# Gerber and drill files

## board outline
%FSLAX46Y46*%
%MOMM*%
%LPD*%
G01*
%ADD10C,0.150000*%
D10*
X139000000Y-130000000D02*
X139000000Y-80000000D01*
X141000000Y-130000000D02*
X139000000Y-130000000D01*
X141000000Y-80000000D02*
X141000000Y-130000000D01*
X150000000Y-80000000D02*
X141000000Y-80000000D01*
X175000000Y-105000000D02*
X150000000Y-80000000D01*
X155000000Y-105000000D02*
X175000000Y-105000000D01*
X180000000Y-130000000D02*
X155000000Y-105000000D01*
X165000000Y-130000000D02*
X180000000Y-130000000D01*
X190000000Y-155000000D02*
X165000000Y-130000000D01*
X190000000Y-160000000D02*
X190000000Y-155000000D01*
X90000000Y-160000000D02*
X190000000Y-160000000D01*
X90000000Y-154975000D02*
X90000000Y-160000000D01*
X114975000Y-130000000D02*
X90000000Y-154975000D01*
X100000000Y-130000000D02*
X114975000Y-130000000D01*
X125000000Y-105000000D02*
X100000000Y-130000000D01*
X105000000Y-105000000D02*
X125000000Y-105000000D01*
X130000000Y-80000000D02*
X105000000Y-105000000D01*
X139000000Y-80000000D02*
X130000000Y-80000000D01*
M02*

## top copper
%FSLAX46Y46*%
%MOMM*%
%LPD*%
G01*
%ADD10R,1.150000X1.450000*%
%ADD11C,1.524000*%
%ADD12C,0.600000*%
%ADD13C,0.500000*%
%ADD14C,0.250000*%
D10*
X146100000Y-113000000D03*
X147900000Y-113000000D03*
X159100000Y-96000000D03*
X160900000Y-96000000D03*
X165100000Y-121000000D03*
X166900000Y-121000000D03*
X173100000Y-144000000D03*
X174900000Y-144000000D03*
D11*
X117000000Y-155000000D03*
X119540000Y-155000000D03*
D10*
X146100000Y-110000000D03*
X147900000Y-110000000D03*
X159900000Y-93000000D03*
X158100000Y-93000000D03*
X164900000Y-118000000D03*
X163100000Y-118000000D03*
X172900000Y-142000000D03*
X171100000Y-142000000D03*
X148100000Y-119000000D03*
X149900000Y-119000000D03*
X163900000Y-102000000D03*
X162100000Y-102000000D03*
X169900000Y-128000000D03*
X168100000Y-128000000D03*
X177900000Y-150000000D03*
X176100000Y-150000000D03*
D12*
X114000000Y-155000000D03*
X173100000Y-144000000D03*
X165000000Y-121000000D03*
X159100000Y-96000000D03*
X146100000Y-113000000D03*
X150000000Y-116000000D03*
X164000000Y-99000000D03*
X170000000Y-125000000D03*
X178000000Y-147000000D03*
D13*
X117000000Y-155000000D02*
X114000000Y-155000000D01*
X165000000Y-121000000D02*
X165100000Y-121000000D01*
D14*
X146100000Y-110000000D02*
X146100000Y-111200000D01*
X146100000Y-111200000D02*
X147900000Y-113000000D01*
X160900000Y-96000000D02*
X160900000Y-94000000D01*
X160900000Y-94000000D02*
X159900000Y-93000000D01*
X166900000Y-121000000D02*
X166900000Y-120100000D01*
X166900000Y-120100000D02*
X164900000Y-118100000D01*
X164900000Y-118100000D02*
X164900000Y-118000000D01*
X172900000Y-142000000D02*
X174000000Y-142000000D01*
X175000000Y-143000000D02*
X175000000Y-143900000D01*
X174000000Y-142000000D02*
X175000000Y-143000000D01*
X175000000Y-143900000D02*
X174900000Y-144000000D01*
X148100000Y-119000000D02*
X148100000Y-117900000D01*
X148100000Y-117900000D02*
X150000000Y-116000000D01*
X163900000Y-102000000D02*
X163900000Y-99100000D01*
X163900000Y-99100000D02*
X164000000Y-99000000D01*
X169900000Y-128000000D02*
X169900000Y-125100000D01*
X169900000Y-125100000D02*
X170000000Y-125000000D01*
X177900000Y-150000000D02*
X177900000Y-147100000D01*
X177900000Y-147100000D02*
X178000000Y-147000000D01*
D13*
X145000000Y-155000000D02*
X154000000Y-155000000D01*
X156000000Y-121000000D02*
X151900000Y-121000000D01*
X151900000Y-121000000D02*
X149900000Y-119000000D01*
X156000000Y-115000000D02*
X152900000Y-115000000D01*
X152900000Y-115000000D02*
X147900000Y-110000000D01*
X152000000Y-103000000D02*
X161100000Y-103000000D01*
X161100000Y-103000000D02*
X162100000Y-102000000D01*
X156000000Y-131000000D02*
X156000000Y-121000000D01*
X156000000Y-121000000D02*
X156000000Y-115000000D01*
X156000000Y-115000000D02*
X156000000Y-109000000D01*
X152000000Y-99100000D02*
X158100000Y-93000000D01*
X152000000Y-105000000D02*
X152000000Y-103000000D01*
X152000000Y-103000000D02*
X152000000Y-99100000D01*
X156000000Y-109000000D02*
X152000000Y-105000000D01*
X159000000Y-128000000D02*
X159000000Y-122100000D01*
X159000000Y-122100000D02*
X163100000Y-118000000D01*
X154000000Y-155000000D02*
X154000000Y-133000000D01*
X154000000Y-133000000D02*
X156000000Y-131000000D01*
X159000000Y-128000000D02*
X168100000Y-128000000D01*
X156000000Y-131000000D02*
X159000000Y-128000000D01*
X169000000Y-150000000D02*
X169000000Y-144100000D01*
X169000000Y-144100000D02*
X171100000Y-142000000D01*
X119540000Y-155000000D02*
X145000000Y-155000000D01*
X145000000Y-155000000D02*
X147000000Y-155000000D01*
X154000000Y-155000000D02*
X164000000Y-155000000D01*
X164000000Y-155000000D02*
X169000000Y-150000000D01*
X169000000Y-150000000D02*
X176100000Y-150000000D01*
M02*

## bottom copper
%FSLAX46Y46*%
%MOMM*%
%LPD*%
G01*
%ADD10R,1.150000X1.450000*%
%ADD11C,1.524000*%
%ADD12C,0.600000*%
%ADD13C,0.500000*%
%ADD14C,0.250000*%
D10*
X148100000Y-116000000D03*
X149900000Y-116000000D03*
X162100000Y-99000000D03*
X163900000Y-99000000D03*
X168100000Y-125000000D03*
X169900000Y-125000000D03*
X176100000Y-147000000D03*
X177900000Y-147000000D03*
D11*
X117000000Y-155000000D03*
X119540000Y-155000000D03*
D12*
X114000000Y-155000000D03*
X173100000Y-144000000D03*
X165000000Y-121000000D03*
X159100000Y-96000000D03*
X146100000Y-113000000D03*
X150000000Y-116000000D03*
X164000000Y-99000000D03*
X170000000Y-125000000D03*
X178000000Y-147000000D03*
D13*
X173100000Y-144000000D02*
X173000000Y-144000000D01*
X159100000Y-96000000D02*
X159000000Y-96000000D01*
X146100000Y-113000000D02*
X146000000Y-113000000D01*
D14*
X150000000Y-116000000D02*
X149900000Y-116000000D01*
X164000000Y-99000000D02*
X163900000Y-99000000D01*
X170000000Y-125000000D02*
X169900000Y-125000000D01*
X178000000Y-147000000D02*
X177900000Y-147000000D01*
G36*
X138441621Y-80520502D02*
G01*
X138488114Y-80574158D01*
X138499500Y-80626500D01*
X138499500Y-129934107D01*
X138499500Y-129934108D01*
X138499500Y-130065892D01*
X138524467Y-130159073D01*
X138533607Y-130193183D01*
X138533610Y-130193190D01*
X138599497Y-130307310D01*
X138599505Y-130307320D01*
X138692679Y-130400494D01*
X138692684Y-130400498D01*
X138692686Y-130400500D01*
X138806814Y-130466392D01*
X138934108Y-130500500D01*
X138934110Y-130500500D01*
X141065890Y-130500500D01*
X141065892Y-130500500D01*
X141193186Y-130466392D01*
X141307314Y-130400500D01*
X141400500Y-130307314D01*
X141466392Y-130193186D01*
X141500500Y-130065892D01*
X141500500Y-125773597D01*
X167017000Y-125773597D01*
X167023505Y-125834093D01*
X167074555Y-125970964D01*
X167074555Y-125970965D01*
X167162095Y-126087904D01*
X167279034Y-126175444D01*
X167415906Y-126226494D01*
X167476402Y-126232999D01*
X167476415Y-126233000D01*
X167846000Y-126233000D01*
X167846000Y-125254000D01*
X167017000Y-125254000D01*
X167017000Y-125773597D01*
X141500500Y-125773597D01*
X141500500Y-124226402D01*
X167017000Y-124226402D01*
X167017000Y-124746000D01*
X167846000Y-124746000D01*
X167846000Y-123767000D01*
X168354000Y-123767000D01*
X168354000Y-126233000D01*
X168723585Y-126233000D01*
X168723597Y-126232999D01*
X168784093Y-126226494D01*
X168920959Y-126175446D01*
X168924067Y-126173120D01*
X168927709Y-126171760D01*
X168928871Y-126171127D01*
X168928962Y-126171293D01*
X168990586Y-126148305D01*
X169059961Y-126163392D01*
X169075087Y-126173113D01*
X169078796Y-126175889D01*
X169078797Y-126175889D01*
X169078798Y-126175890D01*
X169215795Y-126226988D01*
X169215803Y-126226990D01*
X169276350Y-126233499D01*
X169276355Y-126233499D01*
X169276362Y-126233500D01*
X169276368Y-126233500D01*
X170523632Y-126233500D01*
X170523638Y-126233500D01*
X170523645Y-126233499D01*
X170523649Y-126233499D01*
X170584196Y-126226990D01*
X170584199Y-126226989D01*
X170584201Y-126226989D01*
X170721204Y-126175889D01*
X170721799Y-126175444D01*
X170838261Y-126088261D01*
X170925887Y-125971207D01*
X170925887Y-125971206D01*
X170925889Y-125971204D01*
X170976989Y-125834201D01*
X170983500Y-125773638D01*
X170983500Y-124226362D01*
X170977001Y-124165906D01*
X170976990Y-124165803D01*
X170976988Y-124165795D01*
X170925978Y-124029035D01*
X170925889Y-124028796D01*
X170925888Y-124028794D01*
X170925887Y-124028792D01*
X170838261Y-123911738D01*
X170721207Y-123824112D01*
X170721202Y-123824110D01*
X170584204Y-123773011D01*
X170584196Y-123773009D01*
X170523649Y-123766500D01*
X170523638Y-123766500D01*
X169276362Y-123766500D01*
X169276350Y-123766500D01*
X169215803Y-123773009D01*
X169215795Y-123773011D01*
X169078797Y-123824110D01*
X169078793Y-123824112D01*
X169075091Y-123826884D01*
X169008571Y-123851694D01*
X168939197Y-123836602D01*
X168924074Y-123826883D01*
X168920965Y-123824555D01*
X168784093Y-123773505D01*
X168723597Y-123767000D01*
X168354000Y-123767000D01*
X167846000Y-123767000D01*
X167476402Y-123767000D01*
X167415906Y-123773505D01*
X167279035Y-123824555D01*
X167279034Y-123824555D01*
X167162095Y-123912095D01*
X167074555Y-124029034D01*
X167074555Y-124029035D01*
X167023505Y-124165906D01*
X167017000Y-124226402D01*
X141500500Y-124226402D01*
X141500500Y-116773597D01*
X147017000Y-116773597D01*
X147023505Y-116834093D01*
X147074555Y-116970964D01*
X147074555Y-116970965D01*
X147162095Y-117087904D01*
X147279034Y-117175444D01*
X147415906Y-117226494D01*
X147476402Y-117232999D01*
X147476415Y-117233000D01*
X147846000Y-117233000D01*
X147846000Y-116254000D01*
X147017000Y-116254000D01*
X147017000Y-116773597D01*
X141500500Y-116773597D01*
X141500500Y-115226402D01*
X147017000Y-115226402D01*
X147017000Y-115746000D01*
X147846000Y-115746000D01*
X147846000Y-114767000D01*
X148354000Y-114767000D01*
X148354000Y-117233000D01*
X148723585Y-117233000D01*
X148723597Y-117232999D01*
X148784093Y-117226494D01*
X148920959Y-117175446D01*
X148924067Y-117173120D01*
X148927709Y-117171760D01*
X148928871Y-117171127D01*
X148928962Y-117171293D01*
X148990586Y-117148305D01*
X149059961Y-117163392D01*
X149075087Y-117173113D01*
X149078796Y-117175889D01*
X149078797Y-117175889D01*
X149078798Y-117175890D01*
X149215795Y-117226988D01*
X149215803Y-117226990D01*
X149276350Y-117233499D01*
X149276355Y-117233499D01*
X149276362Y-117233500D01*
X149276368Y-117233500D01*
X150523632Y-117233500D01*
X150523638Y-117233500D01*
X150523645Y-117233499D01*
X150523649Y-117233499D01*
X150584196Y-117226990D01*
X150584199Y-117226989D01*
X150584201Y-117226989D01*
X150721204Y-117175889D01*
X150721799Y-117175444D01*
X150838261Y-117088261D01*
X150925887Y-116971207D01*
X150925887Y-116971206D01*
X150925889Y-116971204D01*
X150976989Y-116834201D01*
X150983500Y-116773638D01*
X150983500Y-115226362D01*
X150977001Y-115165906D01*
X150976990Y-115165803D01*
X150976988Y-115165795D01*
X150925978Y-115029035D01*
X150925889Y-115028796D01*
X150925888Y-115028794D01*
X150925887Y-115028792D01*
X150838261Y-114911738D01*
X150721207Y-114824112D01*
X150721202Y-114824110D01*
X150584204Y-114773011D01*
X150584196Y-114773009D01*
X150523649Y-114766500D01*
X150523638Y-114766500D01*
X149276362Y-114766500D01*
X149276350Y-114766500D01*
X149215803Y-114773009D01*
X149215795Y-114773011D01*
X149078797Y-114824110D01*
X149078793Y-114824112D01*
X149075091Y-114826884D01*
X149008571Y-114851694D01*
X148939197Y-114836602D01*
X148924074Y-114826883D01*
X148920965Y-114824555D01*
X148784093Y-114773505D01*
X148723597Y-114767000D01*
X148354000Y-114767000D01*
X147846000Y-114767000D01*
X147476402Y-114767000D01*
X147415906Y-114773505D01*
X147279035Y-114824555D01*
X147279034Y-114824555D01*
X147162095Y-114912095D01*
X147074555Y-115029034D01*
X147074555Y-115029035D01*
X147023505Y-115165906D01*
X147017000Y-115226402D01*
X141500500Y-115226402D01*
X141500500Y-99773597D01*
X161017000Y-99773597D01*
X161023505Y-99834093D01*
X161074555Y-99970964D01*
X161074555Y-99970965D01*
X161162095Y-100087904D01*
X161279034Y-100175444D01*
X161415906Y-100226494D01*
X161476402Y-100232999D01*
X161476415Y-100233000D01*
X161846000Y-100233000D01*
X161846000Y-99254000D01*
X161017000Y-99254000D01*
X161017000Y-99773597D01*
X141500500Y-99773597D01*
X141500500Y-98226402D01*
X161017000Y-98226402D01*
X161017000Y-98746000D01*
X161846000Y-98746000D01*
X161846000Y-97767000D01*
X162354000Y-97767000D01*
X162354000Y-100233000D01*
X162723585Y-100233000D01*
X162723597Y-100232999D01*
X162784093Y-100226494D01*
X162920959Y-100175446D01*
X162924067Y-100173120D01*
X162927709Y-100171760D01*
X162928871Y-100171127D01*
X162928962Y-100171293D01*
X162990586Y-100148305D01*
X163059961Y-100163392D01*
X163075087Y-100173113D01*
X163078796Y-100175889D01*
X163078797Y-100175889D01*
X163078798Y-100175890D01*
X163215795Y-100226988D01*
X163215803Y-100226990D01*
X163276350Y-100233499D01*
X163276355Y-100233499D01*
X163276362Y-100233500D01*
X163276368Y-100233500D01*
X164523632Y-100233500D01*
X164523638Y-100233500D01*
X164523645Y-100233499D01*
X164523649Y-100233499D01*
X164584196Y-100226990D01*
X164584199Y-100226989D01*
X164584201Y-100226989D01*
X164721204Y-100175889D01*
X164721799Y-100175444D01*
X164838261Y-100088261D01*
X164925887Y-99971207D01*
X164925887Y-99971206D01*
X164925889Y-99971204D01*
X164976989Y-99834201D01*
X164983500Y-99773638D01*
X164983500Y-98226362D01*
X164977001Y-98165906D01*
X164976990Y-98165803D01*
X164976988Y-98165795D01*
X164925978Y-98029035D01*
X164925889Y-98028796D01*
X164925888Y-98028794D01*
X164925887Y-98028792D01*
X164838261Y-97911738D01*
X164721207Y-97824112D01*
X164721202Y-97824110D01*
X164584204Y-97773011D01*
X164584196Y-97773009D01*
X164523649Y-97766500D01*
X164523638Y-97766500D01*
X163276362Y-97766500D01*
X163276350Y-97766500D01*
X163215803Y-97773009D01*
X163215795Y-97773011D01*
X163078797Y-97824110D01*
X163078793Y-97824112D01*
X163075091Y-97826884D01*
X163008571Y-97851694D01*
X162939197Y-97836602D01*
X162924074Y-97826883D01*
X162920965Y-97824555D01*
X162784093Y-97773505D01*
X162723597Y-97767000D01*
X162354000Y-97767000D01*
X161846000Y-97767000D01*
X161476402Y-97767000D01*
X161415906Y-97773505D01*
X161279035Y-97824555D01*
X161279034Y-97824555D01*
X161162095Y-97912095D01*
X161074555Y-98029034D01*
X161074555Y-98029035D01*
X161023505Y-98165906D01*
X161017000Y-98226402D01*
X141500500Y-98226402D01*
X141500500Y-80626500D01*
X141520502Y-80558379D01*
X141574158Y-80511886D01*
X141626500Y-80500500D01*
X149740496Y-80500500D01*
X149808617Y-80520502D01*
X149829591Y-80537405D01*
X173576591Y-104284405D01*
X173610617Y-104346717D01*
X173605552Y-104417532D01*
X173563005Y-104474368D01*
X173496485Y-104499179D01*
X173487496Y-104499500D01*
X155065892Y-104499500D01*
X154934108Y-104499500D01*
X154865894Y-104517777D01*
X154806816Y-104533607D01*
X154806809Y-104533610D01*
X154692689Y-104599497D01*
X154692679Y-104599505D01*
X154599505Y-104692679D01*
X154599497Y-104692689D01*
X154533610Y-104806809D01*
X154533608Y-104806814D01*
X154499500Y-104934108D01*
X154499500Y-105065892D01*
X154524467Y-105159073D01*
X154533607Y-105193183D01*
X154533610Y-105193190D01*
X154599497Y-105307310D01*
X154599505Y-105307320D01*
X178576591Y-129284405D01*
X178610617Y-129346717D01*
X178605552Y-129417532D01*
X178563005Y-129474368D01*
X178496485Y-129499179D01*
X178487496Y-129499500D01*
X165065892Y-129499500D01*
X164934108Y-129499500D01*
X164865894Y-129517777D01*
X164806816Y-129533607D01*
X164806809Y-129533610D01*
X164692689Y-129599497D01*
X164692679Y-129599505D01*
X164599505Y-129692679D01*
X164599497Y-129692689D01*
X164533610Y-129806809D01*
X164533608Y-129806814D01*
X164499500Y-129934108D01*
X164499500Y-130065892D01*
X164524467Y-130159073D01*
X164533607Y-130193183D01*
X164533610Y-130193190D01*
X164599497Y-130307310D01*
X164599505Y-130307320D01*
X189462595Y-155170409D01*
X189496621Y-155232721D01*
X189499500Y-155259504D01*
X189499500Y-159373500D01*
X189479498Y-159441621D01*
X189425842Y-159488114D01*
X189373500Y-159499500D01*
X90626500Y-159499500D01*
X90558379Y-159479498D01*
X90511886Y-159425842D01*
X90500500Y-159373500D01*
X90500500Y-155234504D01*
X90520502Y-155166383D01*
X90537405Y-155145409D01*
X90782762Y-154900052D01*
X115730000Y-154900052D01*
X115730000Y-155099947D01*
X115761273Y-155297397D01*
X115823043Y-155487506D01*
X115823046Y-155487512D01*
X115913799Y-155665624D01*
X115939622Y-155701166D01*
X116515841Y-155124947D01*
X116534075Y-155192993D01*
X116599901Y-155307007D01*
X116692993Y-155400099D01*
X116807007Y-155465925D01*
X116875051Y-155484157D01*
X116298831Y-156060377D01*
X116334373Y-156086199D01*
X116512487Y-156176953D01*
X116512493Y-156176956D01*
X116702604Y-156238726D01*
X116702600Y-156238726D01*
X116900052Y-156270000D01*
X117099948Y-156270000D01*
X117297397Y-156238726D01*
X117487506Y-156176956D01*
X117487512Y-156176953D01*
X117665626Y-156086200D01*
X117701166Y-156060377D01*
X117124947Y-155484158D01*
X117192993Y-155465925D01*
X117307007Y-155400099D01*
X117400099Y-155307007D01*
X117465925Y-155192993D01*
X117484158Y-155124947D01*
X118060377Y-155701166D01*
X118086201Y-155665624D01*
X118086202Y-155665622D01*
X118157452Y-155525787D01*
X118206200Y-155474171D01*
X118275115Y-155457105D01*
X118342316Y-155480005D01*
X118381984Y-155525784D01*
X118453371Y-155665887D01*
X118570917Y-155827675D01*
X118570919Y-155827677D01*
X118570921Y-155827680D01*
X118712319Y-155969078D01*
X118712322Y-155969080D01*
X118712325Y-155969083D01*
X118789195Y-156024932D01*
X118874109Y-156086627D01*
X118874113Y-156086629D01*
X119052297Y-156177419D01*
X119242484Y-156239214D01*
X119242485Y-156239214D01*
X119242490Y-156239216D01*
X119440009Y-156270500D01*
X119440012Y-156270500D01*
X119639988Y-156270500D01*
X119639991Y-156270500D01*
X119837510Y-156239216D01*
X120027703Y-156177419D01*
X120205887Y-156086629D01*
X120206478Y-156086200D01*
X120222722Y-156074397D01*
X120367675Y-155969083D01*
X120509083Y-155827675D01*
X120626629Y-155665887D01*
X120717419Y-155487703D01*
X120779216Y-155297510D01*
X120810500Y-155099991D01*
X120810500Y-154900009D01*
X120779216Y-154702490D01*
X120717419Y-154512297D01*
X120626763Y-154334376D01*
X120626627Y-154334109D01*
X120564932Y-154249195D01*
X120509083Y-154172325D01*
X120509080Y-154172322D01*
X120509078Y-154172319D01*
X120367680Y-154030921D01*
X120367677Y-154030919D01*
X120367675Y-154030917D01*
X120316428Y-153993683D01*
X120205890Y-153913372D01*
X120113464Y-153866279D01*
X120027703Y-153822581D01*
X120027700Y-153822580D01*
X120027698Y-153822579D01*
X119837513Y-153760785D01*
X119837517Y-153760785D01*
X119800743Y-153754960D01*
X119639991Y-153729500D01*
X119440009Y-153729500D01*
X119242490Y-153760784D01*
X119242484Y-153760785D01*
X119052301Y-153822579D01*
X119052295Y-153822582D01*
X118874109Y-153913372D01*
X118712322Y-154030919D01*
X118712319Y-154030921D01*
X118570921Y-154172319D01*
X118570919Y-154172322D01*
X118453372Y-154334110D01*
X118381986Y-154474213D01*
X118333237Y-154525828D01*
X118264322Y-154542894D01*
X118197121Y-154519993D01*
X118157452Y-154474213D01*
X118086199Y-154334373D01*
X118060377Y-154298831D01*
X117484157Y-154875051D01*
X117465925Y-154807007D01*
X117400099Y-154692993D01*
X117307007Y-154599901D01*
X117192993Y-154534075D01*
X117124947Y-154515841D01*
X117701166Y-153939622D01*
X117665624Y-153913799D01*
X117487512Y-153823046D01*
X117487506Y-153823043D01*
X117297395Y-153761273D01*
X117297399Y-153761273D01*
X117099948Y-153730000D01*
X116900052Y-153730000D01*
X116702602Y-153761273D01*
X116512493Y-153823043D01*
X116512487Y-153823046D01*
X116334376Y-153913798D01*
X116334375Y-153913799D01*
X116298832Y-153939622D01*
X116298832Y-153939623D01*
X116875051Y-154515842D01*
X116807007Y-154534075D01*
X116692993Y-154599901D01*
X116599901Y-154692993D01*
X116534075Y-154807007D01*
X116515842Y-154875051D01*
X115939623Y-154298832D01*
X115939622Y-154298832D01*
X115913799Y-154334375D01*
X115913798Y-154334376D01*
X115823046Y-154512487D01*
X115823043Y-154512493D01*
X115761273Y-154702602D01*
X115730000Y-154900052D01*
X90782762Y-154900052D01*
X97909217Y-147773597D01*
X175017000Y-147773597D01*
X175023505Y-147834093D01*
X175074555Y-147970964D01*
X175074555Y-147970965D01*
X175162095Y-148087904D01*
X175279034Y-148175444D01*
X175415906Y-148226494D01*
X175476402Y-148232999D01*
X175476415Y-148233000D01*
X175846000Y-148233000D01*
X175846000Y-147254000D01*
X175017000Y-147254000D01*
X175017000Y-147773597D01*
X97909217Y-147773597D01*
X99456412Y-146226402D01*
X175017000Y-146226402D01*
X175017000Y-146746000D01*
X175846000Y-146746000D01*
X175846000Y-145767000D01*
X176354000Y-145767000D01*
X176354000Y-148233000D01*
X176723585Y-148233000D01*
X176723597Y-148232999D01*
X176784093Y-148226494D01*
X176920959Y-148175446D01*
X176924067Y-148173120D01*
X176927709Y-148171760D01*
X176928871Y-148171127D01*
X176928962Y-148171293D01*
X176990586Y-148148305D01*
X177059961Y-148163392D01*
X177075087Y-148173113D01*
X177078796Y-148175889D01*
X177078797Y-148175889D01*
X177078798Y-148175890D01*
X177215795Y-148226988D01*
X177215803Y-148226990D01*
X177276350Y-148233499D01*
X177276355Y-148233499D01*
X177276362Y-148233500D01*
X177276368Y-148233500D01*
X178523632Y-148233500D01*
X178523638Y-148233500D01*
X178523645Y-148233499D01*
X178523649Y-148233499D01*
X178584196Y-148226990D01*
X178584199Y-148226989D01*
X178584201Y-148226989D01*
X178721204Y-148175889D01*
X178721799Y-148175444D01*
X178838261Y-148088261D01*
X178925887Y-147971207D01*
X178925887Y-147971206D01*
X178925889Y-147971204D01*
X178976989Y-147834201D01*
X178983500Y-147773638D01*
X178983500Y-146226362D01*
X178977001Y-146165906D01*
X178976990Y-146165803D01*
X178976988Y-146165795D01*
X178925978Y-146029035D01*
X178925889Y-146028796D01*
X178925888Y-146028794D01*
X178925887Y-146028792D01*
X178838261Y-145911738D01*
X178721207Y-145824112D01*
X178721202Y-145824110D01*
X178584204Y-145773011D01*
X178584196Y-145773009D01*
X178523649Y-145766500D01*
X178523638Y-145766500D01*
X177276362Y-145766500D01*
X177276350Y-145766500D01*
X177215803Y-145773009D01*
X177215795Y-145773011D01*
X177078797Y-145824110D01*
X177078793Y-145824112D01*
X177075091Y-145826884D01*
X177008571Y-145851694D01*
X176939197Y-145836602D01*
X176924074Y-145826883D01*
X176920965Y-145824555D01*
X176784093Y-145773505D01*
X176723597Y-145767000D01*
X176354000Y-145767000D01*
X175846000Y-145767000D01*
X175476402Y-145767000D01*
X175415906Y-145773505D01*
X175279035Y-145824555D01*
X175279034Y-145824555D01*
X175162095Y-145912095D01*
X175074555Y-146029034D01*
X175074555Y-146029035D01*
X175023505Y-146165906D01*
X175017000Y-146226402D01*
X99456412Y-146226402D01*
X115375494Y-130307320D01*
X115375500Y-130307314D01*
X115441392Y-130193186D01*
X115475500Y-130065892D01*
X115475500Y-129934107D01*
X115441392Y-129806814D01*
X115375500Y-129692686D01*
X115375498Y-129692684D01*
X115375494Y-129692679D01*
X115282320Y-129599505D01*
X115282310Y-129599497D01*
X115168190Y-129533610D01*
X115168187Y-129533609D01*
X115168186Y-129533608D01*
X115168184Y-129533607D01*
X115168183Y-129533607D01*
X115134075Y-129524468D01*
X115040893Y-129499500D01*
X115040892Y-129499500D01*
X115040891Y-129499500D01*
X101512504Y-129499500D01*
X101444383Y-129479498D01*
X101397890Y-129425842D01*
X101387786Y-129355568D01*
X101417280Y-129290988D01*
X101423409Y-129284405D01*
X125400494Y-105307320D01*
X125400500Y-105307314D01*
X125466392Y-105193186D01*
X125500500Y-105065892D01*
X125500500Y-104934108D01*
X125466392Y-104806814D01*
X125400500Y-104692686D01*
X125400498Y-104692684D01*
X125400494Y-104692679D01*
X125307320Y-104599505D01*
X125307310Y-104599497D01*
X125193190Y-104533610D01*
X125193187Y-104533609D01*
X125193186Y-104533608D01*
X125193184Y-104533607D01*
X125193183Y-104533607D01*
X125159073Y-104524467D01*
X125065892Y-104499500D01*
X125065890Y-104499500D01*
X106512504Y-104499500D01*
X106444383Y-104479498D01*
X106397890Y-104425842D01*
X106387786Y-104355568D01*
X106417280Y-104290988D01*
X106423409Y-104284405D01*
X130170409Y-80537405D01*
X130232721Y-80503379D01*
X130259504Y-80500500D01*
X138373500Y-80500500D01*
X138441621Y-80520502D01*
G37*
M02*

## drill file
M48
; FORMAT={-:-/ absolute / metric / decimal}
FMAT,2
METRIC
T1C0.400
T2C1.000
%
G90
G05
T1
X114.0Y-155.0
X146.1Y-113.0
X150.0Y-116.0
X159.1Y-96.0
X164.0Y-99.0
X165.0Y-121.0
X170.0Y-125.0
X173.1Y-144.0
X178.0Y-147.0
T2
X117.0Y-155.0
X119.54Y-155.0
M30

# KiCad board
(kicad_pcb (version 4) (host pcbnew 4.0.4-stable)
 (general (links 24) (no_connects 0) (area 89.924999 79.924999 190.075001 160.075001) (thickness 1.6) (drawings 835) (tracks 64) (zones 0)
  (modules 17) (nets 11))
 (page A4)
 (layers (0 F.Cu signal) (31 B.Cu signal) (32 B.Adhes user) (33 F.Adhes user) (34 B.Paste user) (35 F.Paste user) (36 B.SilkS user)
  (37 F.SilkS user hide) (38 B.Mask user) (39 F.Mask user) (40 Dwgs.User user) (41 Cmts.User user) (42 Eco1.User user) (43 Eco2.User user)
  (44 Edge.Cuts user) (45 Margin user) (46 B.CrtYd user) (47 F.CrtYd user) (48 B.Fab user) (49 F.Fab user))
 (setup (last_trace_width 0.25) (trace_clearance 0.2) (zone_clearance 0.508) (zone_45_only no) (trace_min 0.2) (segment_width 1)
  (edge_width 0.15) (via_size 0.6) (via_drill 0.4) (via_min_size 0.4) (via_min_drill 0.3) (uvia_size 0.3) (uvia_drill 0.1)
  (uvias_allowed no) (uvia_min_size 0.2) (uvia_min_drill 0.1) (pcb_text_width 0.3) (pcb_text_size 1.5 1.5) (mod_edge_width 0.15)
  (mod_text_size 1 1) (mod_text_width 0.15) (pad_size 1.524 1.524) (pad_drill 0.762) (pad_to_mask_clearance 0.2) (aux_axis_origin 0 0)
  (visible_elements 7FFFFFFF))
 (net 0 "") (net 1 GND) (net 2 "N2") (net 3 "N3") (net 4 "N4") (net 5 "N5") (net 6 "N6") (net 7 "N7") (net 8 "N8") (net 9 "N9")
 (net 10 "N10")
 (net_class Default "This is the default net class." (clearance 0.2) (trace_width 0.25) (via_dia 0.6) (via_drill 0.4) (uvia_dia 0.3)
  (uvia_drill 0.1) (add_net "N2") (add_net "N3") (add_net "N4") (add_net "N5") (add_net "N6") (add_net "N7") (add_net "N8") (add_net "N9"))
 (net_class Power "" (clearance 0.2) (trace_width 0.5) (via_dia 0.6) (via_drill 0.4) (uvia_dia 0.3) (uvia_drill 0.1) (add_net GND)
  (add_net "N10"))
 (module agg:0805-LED (layer F.Cu) (at 147 113)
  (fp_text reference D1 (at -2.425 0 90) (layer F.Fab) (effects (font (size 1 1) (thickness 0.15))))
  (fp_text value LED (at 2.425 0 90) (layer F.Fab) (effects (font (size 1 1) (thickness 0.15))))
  (pad 1 smd rect (at -0.9 0) (size 1.15 1.45) (layers F.Cu F.Paste F.Mask) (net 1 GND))
  (pad 2 smd rect (at 0.9 0) (size 1.15 1.45) (layers F.Cu F.Paste F.Mask) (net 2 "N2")))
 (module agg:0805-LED (layer F.Cu) (at 160 96)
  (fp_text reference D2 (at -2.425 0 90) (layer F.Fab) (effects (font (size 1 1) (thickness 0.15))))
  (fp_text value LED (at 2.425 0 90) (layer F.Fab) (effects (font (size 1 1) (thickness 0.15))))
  (pad 1 smd rect (at -0.9 0) (size 1.15 1.45) (layers F.Cu F.Paste F.Mask) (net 1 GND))
  (pad 2 smd rect (at 0.9 0) (size 1.15 1.45) (layers F.Cu F.Paste F.Mask) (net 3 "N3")))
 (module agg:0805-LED (layer F.Cu) (at 166 121)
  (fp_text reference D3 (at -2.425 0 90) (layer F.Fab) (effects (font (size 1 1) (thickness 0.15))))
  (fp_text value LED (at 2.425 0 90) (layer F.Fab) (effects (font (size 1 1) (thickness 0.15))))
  (pad 1 smd rect (at -0.9 0) (size 1.15 1.45) (layers F.Cu F.Paste F.Mask) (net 1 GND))
  (pad 2 smd rect (at 0.9 0) (size 1.15 1.45) (layers F.Cu F.Paste F.Mask) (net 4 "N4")))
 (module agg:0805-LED (layer F.Cu) (at 174 144)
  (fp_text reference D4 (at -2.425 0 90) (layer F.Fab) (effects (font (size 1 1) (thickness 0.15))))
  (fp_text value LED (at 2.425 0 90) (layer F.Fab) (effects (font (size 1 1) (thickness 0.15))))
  (pad 1 smd rect (at -0.9 0) (size 1.15 1.45) (layers F.Cu F.Paste F.Mask) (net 1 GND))
  (pad 2 smd rect (at 0.9 0) (size 1.15 1.45) (layers F.Cu F.Paste F.Mask) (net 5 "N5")))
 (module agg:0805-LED (layer B.Cu) (at 149 116)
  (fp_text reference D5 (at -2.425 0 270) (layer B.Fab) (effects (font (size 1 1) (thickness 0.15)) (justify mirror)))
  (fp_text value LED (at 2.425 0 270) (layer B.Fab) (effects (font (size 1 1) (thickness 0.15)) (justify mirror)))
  (pad 1 smd rect (at -0.9 0) (size 1.15 1.45) (layers B.Cu B.Paste B.Mask) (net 1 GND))
  (pad 2 smd rect (at 0.9 0) (size 1.15 1.45) (layers B.Cu B.Paste B.Mask) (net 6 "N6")))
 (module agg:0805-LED (layer B.Cu) (at 163 99)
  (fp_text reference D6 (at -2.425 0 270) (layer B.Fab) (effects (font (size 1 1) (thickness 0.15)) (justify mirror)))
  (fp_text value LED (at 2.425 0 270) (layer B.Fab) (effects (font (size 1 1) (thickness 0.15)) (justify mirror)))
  (pad 1 smd rect (at -0.9 0) (size 1.15 1.45) (layers B.Cu B.Paste B.Mask) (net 1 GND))
  (pad 2 smd rect (at 0.9 0) (size 1.15 1.45) (layers B.Cu B.Paste B.Mask) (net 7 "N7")))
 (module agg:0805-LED (layer B.Cu) (at 169 125)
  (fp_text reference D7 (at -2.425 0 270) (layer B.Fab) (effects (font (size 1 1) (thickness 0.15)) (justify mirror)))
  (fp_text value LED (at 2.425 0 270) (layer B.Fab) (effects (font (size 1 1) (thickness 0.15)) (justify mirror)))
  (pad 1 smd rect (at -0.9 0) (size 1.15 1.45) (layers B.Cu B.Paste B.Mask) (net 1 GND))
  (pad 2 smd rect (at 0.9 0) (size 1.15 1.45) (layers B.Cu B.Paste B.Mask) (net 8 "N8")))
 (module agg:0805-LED (layer B.Cu) (at 177 147)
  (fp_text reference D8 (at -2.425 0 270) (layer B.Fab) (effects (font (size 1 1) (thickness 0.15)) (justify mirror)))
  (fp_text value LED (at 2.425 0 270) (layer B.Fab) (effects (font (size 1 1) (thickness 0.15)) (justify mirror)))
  (pad 1 smd rect (at -0.9 0) (size 1.15 1.45) (layers B.Cu B.Paste B.Mask) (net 1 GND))
  (pad 2 smd rect (at 0.9 0) (size 1.15 1.45) (layers B.Cu B.Paste B.Mask) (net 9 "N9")))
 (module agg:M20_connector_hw (layer F.Cu) (at 117 155)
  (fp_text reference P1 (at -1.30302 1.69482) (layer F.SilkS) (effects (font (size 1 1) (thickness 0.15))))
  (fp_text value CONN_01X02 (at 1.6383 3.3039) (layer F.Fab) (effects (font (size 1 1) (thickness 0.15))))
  (pad 1 thru_hole circle (at 0 0) (size 1.524 1.524) (drill 1) (layers *.Cu *.Mask) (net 1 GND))
  (pad 2 thru_hole circle (at 2.54 0) (size 1.524 1.524) (drill 1) (layers *.Cu *.Mask) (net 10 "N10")))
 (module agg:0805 (layer F.Cu) (at 147 110)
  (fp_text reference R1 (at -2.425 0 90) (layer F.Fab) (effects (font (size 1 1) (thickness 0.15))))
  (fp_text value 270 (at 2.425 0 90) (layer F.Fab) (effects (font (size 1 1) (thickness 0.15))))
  (pad 1 smd rect (at -0.9 0) (size 1.15 1.45) (layers F.Cu F.Paste F.Mask) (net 2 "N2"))
  (pad 2 smd rect (at 0.9 0) (size 1.15 1.45) (layers F.Cu F.Paste F.Mask) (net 10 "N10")))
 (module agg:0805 (layer F.Cu) (at 159 93 180)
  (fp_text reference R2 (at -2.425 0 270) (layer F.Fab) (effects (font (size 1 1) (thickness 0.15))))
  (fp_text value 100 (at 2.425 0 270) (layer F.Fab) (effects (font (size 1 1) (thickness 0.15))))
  (pad 1 smd rect (at -0.9 0 180) (size 1.15 1.45) (layers F.Cu F.Paste F.Mask) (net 3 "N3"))
  (pad 2 smd rect (at 0.9 0 180) (size 1.15 1.45) (layers F.Cu F.Paste F.Mask) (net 10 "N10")))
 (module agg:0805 (layer F.Cu) (at 164 118 180)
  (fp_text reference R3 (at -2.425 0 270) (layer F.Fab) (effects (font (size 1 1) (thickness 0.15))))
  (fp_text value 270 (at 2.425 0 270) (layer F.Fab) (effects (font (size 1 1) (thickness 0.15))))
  (pad 1 smd rect (at -0.9 0 180) (size 1.15 1.45) (layers F.Cu F.Paste F.Mask) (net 4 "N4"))
  (pad 2 smd rect (at 0.9 0 180) (size 1.15 1.45) (layers F.Cu F.Paste F.Mask) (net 10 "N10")))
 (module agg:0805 (layer F.Cu) (at 172 142 180)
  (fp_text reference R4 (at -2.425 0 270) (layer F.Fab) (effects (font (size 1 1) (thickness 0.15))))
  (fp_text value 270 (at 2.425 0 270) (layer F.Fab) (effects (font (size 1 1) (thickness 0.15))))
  (pad 1 smd rect (at -0.9 0 180) (size 1.15 1.45) (layers F.Cu F.Paste F.Mask) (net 5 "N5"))
  (pad 2 smd rect (at 0.9 0 180) (size 1.15 1.45) (layers F.Cu F.Paste F.Mask) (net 10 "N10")))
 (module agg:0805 (layer F.Cu) (at 149 119)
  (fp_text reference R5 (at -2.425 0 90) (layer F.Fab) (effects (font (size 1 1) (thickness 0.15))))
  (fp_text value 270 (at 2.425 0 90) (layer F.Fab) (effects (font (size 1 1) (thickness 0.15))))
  (pad 1 smd rect (at -0.9 0) (size 1.15 1.45) (layers F.Cu F.Paste F.Mask) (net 6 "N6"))
  (pad 2 smd rect (at 0.9 0) (size 1.15 1.45) (layers F.Cu F.Paste F.Mask) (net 10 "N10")))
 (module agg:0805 (layer F.Cu) (at 163 102 180)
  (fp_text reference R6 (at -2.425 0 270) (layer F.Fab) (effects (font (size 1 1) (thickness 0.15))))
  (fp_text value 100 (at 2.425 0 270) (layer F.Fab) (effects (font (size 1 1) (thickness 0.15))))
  (pad 1 smd rect (at -0.9 0 180) (size 1.15 1.45) (layers F.Cu F.Paste F.Mask) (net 7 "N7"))
  (pad 2 smd rect (at 0.9 0 180) (size 1.15 1.45) (layers F.Cu F.Paste F.Mask) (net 10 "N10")))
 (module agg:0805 (layer F.Cu) (at 169 128 180)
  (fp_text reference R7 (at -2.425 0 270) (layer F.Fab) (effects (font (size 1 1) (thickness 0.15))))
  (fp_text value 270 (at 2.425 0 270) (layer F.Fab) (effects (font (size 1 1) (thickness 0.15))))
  (pad 1 smd rect (at -0.9 0 180) (size 1.15 1.45) (layers F.Cu F.Paste F.Mask) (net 8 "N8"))
  (pad 2 smd rect (at 0.9 0 180) (size 1.15 1.45) (layers F.Cu F.Paste F.Mask) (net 10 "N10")))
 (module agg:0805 (layer F.Cu) (at 177 150 180)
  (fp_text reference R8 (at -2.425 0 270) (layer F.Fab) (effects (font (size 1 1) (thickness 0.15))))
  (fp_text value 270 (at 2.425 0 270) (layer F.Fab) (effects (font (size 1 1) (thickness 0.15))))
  (pad 1 smd rect (at -0.9 0 180) (size 1.15 1.45) (layers F.Cu F.Paste F.Mask) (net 9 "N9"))
  (pad 2 smd rect (at 0.9 0 180) (size 1.15 1.45) (layers F.Cu F.Paste F.Mask) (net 10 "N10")))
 (gr_line (start 139 130) (end 139 80) (angle 90) (layer Edge.Cuts) (width 0.15))
 (gr_line (start 141 130) (end 139 130) (angle 90) (layer Edge.Cuts) (width 0.15))
 (gr_line (start 141 80) (end 141 130) (angle 90) (layer Edge.Cuts) (width 0.15))
 (gr_line (start 150 80) (end 141 80) (angle 90) (layer Edge.Cuts) (width 0.15))
 (gr_line (start 175 105) (end 150 80) (angle 90) (layer Edge.Cuts) (width 0.15))
 (gr_line (start 155 105) (end 175 105) (angle 90) (layer Edge.Cuts) (width 0.15))
 (gr_line (start 180 130) (end 155 105) (angle 90) (layer Edge.Cuts) (width 0.15))
 (gr_line (start 165 130) (end 180 130) (angle 90) (layer Edge.Cuts) (width 0.15))
 (gr_line (start 190 155) (end 165 130) (angle 90) (layer Edge.Cuts) (width 0.15))
 (gr_line (start 190 160) (end 190 155) (angle 90) (layer Edge.Cuts) (width 0.15))
 (gr_line (start 90 160) (end 190 160) (angle 90) (layer Edge.Cuts) (width 0.15))
 (gr_line (start 90 154.975) (end 90 160) (angle 90) (layer Edge.Cuts) (width 0.15))
 (gr_line (start 114.975 130) (end 90 154.975) (angle 90) (layer Edge.Cuts) (width 0.15))
 (gr_line (start 100 130) (end 114.975 130) (angle 90) (layer Edge.Cuts) (width 0.15))
 (gr_line (start 125 105) (end 100 130) (angle 90) (layer Edge.Cuts) (width 0.15))
 (gr_line (start 105 105) (end 125 105) (angle 90) (layer Edge.Cuts) (width 0.15))
 (gr_line (start 130 80) (end 105 105) (angle 90) (layer Edge.Cuts) (width 0.15))
 (gr_line (start 139 80) (end 130 80) (angle 90) (layer Edge.Cuts) (width 0.15))
 (segment (start 117 155) (end 114 155) (width 0.5) (layer F.Cu) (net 1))
 (via (at 114 155) (size 0.6) (drill 0.4) (layers F.Cu B.Cu) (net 1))
 (via (at 173.1 144) (size 0.6) (drill 0.4) (layers F.Cu B.Cu) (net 1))
 (segment (start 173.1 144) (end 173 144) (width 0.5) (layer B.Cu) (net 1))
 (via (at 165 121) (size 0.6) (drill 0.4) (layers F.Cu B.Cu) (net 1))
 (segment (start 165 121) (end 165.1 121) (width 0.5) (layer F.Cu) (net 1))
 (via (at 159.1 96) (size 0.6) (drill 0.4) (layers F.Cu B.Cu) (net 1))
 (segment (start 159.1 96) (end 159 96) (width 0.5) (layer B.Cu) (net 1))
 (via (at 146.1 113) (size 0.6) (drill 0.4) (layers F.Cu B.Cu) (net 1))
 (segment (start 146.1 113) (end 146 113) (width 0.5) (layer B.Cu) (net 1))
 (segment (start 146.1 110) (end 146.1 111.2) (width 0.25) (layer F.Cu) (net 2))
 (segment (start 146.1 111.2) (end 147.9 113) (width 0.25) (layer F.Cu) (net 2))
 (segment (start 160.9 96) (end 160.9 94) (width 0.25) (layer F.Cu) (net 3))
 (segment (start 160.9 94) (end 159.9 93) (width 0.25) (layer F.Cu) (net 3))
 (segment (start 166.9 121) (end 166.9 120.1) (width 0.25) (layer F.Cu) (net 4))
 (segment (start 166.9 120.1) (end 164.9 118.1) (width 0.25) (layer F.Cu) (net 4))
 (segment (start 164.9 118.1) (end 164.9 118) (width 0.25) (layer F.Cu) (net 4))
 (segment (start 172.9 142) (end 174 142) (width 0.25) (layer F.Cu) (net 5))
 (segment (start 175 143) (end 175 143.9) (width 0.25) (layer F.Cu) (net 5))
 (segment (start 174 142) (end 175 143) (width 0.25) (layer F.Cu) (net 5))
 (segment (start 175 143.9) (end 174.9 144) (width 0.25) (layer F.Cu) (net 5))
 (segment (start 148.1 119) (end 148.1 117.9) (width 0.25) (layer F.Cu) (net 6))
 (segment (start 150 116) (end 149.9 116) (width 0.25) (layer B.Cu) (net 6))
 (via (at 150 116) (size 0.6) (drill 0.4) (layers F.Cu B.Cu) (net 6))
 (segment (start 148.1 117.9) (end 150 116) (width 0.25) (layer F.Cu) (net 6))
 (segment (start 163.9 102) (end 163.9 99.1) (width 0.25) (layer F.Cu) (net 7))
 (segment (start 164 99) (end 163.9 99) (width 0.25) (layer B.Cu) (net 7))
 (via (at 164 99) (size 0.6) (drill 0.4) (layers F.Cu B.Cu) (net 7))
 (segment (start 163.9 99.1) (end 164 99) (width 0.25) (layer F.Cu) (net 7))
 (segment (start 169.9 128) (end 169.9 125.1) (width 0.25) (layer F.Cu) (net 8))
 (segment (start 170 125) (end 169.9 125) (width 0.25) (layer B.Cu) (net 8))
 (via (at 170 125) (size 0.6) (drill 0.4) (layers F.Cu B.Cu) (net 8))
 (segment (start 169.9 125.1) (end 170 125) (width 0.25) (layer F.Cu) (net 8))
 (segment (start 177.9 150) (end 177.9 147.1) (width 0.25) (layer F.Cu) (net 9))
 (segment (start 178 147) (end 177.9 147) (width 0.25) (layer B.Cu) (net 9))
 (via (at 178 147) (size 0.6) (drill 0.4) (layers F.Cu B.Cu) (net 9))
 (segment (start 177.9 147.1) (end 178 147) (width 0.25) (layer F.Cu) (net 9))
 (segment (start 145 155) (end 154 155) (width 0.5) (layer F.Cu) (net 10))
 (segment (start 156 121) (end 151.9 121) (width 0.5) (layer F.Cu) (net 10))
 (segment (start 151.9 121) (end 149.9 119) (width 0.5) (layer F.Cu) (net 10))
 (segment (start 156 115) (end 152.9 115) (width 0.5) (layer F.Cu) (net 10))
 (segment (start 152.9 115) (end 147.9 110) (width 0.5) (layer F.Cu) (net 10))
 (segment (start 152 103) (end 161.1 103) (width 0.5) (layer F.Cu) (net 10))
 (segment (start 161.1 103) (end 162.1 102) (width 0.5) (layer F.Cu) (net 10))
 (segment (start 156 131) (end 156 121) (width 0.5) (layer F.Cu) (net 10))
 (segment (start 156 121) (end 156 115) (width 0.5) (layer F.Cu) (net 10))
 (segment (start 156 115) (end 156 109) (width 0.5) (layer F.Cu) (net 10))
 (segment (start 152 99.1) (end 158.1 93) (width 0.5) (layer F.Cu) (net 10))
 (segment (start 152 105) (end 152 103) (width 0.5) (layer F.Cu) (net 10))
 (segment (start 152 103) (end 152 99.1) (width 0.5) (layer F.Cu) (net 10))
 (segment (start 156 109) (end 152 105) (width 0.5) (layer F.Cu) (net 10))
 (segment (start 159 128) (end 159 122.1) (width 0.5) (layer F.Cu) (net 10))
 (segment (start 159 122.1) (end 163.1 118) (width 0.5) (layer F.Cu) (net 10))
 (segment (start 154 155) (end 154 133) (width 0.5) (layer F.Cu) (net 10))
 (segment (start 154 133) (end 156 131) (width 0.5) (layer F.Cu) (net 10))
 (segment (start 159 128) (end 168.1 128) (width 0.5) (layer F.Cu) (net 10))
 (segment (start 156 131) (end 159 128) (width 0.5) (layer F.Cu) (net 10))
 (segment (start 169 150) (end 169 144.1) (width 0.5) (layer F.Cu) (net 10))
 (segment (start 169 144.1) (end 171.1 142) (width 0.5) (layer F.Cu) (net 10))
 (segment (start 119.54 155) (end 145 155) (width 0.5) (layer F.Cu) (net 10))
 (segment (start 145 155) (end 147 155) (width 0.5) (layer F.Cu) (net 10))
 (segment (start 154 155) (end 164 155) (width 0.5) (layer F.Cu) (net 10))
 (segment (start 164 155) (end 169 150) (width 0.5) (layer F.Cu) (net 10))
 (segment (start 169 150) (end 176.1 150) (width 0.5) (layer F.Cu) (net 10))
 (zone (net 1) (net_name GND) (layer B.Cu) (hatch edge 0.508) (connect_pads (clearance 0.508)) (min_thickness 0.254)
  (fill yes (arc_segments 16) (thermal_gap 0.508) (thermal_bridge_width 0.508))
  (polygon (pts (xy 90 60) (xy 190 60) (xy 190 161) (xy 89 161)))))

